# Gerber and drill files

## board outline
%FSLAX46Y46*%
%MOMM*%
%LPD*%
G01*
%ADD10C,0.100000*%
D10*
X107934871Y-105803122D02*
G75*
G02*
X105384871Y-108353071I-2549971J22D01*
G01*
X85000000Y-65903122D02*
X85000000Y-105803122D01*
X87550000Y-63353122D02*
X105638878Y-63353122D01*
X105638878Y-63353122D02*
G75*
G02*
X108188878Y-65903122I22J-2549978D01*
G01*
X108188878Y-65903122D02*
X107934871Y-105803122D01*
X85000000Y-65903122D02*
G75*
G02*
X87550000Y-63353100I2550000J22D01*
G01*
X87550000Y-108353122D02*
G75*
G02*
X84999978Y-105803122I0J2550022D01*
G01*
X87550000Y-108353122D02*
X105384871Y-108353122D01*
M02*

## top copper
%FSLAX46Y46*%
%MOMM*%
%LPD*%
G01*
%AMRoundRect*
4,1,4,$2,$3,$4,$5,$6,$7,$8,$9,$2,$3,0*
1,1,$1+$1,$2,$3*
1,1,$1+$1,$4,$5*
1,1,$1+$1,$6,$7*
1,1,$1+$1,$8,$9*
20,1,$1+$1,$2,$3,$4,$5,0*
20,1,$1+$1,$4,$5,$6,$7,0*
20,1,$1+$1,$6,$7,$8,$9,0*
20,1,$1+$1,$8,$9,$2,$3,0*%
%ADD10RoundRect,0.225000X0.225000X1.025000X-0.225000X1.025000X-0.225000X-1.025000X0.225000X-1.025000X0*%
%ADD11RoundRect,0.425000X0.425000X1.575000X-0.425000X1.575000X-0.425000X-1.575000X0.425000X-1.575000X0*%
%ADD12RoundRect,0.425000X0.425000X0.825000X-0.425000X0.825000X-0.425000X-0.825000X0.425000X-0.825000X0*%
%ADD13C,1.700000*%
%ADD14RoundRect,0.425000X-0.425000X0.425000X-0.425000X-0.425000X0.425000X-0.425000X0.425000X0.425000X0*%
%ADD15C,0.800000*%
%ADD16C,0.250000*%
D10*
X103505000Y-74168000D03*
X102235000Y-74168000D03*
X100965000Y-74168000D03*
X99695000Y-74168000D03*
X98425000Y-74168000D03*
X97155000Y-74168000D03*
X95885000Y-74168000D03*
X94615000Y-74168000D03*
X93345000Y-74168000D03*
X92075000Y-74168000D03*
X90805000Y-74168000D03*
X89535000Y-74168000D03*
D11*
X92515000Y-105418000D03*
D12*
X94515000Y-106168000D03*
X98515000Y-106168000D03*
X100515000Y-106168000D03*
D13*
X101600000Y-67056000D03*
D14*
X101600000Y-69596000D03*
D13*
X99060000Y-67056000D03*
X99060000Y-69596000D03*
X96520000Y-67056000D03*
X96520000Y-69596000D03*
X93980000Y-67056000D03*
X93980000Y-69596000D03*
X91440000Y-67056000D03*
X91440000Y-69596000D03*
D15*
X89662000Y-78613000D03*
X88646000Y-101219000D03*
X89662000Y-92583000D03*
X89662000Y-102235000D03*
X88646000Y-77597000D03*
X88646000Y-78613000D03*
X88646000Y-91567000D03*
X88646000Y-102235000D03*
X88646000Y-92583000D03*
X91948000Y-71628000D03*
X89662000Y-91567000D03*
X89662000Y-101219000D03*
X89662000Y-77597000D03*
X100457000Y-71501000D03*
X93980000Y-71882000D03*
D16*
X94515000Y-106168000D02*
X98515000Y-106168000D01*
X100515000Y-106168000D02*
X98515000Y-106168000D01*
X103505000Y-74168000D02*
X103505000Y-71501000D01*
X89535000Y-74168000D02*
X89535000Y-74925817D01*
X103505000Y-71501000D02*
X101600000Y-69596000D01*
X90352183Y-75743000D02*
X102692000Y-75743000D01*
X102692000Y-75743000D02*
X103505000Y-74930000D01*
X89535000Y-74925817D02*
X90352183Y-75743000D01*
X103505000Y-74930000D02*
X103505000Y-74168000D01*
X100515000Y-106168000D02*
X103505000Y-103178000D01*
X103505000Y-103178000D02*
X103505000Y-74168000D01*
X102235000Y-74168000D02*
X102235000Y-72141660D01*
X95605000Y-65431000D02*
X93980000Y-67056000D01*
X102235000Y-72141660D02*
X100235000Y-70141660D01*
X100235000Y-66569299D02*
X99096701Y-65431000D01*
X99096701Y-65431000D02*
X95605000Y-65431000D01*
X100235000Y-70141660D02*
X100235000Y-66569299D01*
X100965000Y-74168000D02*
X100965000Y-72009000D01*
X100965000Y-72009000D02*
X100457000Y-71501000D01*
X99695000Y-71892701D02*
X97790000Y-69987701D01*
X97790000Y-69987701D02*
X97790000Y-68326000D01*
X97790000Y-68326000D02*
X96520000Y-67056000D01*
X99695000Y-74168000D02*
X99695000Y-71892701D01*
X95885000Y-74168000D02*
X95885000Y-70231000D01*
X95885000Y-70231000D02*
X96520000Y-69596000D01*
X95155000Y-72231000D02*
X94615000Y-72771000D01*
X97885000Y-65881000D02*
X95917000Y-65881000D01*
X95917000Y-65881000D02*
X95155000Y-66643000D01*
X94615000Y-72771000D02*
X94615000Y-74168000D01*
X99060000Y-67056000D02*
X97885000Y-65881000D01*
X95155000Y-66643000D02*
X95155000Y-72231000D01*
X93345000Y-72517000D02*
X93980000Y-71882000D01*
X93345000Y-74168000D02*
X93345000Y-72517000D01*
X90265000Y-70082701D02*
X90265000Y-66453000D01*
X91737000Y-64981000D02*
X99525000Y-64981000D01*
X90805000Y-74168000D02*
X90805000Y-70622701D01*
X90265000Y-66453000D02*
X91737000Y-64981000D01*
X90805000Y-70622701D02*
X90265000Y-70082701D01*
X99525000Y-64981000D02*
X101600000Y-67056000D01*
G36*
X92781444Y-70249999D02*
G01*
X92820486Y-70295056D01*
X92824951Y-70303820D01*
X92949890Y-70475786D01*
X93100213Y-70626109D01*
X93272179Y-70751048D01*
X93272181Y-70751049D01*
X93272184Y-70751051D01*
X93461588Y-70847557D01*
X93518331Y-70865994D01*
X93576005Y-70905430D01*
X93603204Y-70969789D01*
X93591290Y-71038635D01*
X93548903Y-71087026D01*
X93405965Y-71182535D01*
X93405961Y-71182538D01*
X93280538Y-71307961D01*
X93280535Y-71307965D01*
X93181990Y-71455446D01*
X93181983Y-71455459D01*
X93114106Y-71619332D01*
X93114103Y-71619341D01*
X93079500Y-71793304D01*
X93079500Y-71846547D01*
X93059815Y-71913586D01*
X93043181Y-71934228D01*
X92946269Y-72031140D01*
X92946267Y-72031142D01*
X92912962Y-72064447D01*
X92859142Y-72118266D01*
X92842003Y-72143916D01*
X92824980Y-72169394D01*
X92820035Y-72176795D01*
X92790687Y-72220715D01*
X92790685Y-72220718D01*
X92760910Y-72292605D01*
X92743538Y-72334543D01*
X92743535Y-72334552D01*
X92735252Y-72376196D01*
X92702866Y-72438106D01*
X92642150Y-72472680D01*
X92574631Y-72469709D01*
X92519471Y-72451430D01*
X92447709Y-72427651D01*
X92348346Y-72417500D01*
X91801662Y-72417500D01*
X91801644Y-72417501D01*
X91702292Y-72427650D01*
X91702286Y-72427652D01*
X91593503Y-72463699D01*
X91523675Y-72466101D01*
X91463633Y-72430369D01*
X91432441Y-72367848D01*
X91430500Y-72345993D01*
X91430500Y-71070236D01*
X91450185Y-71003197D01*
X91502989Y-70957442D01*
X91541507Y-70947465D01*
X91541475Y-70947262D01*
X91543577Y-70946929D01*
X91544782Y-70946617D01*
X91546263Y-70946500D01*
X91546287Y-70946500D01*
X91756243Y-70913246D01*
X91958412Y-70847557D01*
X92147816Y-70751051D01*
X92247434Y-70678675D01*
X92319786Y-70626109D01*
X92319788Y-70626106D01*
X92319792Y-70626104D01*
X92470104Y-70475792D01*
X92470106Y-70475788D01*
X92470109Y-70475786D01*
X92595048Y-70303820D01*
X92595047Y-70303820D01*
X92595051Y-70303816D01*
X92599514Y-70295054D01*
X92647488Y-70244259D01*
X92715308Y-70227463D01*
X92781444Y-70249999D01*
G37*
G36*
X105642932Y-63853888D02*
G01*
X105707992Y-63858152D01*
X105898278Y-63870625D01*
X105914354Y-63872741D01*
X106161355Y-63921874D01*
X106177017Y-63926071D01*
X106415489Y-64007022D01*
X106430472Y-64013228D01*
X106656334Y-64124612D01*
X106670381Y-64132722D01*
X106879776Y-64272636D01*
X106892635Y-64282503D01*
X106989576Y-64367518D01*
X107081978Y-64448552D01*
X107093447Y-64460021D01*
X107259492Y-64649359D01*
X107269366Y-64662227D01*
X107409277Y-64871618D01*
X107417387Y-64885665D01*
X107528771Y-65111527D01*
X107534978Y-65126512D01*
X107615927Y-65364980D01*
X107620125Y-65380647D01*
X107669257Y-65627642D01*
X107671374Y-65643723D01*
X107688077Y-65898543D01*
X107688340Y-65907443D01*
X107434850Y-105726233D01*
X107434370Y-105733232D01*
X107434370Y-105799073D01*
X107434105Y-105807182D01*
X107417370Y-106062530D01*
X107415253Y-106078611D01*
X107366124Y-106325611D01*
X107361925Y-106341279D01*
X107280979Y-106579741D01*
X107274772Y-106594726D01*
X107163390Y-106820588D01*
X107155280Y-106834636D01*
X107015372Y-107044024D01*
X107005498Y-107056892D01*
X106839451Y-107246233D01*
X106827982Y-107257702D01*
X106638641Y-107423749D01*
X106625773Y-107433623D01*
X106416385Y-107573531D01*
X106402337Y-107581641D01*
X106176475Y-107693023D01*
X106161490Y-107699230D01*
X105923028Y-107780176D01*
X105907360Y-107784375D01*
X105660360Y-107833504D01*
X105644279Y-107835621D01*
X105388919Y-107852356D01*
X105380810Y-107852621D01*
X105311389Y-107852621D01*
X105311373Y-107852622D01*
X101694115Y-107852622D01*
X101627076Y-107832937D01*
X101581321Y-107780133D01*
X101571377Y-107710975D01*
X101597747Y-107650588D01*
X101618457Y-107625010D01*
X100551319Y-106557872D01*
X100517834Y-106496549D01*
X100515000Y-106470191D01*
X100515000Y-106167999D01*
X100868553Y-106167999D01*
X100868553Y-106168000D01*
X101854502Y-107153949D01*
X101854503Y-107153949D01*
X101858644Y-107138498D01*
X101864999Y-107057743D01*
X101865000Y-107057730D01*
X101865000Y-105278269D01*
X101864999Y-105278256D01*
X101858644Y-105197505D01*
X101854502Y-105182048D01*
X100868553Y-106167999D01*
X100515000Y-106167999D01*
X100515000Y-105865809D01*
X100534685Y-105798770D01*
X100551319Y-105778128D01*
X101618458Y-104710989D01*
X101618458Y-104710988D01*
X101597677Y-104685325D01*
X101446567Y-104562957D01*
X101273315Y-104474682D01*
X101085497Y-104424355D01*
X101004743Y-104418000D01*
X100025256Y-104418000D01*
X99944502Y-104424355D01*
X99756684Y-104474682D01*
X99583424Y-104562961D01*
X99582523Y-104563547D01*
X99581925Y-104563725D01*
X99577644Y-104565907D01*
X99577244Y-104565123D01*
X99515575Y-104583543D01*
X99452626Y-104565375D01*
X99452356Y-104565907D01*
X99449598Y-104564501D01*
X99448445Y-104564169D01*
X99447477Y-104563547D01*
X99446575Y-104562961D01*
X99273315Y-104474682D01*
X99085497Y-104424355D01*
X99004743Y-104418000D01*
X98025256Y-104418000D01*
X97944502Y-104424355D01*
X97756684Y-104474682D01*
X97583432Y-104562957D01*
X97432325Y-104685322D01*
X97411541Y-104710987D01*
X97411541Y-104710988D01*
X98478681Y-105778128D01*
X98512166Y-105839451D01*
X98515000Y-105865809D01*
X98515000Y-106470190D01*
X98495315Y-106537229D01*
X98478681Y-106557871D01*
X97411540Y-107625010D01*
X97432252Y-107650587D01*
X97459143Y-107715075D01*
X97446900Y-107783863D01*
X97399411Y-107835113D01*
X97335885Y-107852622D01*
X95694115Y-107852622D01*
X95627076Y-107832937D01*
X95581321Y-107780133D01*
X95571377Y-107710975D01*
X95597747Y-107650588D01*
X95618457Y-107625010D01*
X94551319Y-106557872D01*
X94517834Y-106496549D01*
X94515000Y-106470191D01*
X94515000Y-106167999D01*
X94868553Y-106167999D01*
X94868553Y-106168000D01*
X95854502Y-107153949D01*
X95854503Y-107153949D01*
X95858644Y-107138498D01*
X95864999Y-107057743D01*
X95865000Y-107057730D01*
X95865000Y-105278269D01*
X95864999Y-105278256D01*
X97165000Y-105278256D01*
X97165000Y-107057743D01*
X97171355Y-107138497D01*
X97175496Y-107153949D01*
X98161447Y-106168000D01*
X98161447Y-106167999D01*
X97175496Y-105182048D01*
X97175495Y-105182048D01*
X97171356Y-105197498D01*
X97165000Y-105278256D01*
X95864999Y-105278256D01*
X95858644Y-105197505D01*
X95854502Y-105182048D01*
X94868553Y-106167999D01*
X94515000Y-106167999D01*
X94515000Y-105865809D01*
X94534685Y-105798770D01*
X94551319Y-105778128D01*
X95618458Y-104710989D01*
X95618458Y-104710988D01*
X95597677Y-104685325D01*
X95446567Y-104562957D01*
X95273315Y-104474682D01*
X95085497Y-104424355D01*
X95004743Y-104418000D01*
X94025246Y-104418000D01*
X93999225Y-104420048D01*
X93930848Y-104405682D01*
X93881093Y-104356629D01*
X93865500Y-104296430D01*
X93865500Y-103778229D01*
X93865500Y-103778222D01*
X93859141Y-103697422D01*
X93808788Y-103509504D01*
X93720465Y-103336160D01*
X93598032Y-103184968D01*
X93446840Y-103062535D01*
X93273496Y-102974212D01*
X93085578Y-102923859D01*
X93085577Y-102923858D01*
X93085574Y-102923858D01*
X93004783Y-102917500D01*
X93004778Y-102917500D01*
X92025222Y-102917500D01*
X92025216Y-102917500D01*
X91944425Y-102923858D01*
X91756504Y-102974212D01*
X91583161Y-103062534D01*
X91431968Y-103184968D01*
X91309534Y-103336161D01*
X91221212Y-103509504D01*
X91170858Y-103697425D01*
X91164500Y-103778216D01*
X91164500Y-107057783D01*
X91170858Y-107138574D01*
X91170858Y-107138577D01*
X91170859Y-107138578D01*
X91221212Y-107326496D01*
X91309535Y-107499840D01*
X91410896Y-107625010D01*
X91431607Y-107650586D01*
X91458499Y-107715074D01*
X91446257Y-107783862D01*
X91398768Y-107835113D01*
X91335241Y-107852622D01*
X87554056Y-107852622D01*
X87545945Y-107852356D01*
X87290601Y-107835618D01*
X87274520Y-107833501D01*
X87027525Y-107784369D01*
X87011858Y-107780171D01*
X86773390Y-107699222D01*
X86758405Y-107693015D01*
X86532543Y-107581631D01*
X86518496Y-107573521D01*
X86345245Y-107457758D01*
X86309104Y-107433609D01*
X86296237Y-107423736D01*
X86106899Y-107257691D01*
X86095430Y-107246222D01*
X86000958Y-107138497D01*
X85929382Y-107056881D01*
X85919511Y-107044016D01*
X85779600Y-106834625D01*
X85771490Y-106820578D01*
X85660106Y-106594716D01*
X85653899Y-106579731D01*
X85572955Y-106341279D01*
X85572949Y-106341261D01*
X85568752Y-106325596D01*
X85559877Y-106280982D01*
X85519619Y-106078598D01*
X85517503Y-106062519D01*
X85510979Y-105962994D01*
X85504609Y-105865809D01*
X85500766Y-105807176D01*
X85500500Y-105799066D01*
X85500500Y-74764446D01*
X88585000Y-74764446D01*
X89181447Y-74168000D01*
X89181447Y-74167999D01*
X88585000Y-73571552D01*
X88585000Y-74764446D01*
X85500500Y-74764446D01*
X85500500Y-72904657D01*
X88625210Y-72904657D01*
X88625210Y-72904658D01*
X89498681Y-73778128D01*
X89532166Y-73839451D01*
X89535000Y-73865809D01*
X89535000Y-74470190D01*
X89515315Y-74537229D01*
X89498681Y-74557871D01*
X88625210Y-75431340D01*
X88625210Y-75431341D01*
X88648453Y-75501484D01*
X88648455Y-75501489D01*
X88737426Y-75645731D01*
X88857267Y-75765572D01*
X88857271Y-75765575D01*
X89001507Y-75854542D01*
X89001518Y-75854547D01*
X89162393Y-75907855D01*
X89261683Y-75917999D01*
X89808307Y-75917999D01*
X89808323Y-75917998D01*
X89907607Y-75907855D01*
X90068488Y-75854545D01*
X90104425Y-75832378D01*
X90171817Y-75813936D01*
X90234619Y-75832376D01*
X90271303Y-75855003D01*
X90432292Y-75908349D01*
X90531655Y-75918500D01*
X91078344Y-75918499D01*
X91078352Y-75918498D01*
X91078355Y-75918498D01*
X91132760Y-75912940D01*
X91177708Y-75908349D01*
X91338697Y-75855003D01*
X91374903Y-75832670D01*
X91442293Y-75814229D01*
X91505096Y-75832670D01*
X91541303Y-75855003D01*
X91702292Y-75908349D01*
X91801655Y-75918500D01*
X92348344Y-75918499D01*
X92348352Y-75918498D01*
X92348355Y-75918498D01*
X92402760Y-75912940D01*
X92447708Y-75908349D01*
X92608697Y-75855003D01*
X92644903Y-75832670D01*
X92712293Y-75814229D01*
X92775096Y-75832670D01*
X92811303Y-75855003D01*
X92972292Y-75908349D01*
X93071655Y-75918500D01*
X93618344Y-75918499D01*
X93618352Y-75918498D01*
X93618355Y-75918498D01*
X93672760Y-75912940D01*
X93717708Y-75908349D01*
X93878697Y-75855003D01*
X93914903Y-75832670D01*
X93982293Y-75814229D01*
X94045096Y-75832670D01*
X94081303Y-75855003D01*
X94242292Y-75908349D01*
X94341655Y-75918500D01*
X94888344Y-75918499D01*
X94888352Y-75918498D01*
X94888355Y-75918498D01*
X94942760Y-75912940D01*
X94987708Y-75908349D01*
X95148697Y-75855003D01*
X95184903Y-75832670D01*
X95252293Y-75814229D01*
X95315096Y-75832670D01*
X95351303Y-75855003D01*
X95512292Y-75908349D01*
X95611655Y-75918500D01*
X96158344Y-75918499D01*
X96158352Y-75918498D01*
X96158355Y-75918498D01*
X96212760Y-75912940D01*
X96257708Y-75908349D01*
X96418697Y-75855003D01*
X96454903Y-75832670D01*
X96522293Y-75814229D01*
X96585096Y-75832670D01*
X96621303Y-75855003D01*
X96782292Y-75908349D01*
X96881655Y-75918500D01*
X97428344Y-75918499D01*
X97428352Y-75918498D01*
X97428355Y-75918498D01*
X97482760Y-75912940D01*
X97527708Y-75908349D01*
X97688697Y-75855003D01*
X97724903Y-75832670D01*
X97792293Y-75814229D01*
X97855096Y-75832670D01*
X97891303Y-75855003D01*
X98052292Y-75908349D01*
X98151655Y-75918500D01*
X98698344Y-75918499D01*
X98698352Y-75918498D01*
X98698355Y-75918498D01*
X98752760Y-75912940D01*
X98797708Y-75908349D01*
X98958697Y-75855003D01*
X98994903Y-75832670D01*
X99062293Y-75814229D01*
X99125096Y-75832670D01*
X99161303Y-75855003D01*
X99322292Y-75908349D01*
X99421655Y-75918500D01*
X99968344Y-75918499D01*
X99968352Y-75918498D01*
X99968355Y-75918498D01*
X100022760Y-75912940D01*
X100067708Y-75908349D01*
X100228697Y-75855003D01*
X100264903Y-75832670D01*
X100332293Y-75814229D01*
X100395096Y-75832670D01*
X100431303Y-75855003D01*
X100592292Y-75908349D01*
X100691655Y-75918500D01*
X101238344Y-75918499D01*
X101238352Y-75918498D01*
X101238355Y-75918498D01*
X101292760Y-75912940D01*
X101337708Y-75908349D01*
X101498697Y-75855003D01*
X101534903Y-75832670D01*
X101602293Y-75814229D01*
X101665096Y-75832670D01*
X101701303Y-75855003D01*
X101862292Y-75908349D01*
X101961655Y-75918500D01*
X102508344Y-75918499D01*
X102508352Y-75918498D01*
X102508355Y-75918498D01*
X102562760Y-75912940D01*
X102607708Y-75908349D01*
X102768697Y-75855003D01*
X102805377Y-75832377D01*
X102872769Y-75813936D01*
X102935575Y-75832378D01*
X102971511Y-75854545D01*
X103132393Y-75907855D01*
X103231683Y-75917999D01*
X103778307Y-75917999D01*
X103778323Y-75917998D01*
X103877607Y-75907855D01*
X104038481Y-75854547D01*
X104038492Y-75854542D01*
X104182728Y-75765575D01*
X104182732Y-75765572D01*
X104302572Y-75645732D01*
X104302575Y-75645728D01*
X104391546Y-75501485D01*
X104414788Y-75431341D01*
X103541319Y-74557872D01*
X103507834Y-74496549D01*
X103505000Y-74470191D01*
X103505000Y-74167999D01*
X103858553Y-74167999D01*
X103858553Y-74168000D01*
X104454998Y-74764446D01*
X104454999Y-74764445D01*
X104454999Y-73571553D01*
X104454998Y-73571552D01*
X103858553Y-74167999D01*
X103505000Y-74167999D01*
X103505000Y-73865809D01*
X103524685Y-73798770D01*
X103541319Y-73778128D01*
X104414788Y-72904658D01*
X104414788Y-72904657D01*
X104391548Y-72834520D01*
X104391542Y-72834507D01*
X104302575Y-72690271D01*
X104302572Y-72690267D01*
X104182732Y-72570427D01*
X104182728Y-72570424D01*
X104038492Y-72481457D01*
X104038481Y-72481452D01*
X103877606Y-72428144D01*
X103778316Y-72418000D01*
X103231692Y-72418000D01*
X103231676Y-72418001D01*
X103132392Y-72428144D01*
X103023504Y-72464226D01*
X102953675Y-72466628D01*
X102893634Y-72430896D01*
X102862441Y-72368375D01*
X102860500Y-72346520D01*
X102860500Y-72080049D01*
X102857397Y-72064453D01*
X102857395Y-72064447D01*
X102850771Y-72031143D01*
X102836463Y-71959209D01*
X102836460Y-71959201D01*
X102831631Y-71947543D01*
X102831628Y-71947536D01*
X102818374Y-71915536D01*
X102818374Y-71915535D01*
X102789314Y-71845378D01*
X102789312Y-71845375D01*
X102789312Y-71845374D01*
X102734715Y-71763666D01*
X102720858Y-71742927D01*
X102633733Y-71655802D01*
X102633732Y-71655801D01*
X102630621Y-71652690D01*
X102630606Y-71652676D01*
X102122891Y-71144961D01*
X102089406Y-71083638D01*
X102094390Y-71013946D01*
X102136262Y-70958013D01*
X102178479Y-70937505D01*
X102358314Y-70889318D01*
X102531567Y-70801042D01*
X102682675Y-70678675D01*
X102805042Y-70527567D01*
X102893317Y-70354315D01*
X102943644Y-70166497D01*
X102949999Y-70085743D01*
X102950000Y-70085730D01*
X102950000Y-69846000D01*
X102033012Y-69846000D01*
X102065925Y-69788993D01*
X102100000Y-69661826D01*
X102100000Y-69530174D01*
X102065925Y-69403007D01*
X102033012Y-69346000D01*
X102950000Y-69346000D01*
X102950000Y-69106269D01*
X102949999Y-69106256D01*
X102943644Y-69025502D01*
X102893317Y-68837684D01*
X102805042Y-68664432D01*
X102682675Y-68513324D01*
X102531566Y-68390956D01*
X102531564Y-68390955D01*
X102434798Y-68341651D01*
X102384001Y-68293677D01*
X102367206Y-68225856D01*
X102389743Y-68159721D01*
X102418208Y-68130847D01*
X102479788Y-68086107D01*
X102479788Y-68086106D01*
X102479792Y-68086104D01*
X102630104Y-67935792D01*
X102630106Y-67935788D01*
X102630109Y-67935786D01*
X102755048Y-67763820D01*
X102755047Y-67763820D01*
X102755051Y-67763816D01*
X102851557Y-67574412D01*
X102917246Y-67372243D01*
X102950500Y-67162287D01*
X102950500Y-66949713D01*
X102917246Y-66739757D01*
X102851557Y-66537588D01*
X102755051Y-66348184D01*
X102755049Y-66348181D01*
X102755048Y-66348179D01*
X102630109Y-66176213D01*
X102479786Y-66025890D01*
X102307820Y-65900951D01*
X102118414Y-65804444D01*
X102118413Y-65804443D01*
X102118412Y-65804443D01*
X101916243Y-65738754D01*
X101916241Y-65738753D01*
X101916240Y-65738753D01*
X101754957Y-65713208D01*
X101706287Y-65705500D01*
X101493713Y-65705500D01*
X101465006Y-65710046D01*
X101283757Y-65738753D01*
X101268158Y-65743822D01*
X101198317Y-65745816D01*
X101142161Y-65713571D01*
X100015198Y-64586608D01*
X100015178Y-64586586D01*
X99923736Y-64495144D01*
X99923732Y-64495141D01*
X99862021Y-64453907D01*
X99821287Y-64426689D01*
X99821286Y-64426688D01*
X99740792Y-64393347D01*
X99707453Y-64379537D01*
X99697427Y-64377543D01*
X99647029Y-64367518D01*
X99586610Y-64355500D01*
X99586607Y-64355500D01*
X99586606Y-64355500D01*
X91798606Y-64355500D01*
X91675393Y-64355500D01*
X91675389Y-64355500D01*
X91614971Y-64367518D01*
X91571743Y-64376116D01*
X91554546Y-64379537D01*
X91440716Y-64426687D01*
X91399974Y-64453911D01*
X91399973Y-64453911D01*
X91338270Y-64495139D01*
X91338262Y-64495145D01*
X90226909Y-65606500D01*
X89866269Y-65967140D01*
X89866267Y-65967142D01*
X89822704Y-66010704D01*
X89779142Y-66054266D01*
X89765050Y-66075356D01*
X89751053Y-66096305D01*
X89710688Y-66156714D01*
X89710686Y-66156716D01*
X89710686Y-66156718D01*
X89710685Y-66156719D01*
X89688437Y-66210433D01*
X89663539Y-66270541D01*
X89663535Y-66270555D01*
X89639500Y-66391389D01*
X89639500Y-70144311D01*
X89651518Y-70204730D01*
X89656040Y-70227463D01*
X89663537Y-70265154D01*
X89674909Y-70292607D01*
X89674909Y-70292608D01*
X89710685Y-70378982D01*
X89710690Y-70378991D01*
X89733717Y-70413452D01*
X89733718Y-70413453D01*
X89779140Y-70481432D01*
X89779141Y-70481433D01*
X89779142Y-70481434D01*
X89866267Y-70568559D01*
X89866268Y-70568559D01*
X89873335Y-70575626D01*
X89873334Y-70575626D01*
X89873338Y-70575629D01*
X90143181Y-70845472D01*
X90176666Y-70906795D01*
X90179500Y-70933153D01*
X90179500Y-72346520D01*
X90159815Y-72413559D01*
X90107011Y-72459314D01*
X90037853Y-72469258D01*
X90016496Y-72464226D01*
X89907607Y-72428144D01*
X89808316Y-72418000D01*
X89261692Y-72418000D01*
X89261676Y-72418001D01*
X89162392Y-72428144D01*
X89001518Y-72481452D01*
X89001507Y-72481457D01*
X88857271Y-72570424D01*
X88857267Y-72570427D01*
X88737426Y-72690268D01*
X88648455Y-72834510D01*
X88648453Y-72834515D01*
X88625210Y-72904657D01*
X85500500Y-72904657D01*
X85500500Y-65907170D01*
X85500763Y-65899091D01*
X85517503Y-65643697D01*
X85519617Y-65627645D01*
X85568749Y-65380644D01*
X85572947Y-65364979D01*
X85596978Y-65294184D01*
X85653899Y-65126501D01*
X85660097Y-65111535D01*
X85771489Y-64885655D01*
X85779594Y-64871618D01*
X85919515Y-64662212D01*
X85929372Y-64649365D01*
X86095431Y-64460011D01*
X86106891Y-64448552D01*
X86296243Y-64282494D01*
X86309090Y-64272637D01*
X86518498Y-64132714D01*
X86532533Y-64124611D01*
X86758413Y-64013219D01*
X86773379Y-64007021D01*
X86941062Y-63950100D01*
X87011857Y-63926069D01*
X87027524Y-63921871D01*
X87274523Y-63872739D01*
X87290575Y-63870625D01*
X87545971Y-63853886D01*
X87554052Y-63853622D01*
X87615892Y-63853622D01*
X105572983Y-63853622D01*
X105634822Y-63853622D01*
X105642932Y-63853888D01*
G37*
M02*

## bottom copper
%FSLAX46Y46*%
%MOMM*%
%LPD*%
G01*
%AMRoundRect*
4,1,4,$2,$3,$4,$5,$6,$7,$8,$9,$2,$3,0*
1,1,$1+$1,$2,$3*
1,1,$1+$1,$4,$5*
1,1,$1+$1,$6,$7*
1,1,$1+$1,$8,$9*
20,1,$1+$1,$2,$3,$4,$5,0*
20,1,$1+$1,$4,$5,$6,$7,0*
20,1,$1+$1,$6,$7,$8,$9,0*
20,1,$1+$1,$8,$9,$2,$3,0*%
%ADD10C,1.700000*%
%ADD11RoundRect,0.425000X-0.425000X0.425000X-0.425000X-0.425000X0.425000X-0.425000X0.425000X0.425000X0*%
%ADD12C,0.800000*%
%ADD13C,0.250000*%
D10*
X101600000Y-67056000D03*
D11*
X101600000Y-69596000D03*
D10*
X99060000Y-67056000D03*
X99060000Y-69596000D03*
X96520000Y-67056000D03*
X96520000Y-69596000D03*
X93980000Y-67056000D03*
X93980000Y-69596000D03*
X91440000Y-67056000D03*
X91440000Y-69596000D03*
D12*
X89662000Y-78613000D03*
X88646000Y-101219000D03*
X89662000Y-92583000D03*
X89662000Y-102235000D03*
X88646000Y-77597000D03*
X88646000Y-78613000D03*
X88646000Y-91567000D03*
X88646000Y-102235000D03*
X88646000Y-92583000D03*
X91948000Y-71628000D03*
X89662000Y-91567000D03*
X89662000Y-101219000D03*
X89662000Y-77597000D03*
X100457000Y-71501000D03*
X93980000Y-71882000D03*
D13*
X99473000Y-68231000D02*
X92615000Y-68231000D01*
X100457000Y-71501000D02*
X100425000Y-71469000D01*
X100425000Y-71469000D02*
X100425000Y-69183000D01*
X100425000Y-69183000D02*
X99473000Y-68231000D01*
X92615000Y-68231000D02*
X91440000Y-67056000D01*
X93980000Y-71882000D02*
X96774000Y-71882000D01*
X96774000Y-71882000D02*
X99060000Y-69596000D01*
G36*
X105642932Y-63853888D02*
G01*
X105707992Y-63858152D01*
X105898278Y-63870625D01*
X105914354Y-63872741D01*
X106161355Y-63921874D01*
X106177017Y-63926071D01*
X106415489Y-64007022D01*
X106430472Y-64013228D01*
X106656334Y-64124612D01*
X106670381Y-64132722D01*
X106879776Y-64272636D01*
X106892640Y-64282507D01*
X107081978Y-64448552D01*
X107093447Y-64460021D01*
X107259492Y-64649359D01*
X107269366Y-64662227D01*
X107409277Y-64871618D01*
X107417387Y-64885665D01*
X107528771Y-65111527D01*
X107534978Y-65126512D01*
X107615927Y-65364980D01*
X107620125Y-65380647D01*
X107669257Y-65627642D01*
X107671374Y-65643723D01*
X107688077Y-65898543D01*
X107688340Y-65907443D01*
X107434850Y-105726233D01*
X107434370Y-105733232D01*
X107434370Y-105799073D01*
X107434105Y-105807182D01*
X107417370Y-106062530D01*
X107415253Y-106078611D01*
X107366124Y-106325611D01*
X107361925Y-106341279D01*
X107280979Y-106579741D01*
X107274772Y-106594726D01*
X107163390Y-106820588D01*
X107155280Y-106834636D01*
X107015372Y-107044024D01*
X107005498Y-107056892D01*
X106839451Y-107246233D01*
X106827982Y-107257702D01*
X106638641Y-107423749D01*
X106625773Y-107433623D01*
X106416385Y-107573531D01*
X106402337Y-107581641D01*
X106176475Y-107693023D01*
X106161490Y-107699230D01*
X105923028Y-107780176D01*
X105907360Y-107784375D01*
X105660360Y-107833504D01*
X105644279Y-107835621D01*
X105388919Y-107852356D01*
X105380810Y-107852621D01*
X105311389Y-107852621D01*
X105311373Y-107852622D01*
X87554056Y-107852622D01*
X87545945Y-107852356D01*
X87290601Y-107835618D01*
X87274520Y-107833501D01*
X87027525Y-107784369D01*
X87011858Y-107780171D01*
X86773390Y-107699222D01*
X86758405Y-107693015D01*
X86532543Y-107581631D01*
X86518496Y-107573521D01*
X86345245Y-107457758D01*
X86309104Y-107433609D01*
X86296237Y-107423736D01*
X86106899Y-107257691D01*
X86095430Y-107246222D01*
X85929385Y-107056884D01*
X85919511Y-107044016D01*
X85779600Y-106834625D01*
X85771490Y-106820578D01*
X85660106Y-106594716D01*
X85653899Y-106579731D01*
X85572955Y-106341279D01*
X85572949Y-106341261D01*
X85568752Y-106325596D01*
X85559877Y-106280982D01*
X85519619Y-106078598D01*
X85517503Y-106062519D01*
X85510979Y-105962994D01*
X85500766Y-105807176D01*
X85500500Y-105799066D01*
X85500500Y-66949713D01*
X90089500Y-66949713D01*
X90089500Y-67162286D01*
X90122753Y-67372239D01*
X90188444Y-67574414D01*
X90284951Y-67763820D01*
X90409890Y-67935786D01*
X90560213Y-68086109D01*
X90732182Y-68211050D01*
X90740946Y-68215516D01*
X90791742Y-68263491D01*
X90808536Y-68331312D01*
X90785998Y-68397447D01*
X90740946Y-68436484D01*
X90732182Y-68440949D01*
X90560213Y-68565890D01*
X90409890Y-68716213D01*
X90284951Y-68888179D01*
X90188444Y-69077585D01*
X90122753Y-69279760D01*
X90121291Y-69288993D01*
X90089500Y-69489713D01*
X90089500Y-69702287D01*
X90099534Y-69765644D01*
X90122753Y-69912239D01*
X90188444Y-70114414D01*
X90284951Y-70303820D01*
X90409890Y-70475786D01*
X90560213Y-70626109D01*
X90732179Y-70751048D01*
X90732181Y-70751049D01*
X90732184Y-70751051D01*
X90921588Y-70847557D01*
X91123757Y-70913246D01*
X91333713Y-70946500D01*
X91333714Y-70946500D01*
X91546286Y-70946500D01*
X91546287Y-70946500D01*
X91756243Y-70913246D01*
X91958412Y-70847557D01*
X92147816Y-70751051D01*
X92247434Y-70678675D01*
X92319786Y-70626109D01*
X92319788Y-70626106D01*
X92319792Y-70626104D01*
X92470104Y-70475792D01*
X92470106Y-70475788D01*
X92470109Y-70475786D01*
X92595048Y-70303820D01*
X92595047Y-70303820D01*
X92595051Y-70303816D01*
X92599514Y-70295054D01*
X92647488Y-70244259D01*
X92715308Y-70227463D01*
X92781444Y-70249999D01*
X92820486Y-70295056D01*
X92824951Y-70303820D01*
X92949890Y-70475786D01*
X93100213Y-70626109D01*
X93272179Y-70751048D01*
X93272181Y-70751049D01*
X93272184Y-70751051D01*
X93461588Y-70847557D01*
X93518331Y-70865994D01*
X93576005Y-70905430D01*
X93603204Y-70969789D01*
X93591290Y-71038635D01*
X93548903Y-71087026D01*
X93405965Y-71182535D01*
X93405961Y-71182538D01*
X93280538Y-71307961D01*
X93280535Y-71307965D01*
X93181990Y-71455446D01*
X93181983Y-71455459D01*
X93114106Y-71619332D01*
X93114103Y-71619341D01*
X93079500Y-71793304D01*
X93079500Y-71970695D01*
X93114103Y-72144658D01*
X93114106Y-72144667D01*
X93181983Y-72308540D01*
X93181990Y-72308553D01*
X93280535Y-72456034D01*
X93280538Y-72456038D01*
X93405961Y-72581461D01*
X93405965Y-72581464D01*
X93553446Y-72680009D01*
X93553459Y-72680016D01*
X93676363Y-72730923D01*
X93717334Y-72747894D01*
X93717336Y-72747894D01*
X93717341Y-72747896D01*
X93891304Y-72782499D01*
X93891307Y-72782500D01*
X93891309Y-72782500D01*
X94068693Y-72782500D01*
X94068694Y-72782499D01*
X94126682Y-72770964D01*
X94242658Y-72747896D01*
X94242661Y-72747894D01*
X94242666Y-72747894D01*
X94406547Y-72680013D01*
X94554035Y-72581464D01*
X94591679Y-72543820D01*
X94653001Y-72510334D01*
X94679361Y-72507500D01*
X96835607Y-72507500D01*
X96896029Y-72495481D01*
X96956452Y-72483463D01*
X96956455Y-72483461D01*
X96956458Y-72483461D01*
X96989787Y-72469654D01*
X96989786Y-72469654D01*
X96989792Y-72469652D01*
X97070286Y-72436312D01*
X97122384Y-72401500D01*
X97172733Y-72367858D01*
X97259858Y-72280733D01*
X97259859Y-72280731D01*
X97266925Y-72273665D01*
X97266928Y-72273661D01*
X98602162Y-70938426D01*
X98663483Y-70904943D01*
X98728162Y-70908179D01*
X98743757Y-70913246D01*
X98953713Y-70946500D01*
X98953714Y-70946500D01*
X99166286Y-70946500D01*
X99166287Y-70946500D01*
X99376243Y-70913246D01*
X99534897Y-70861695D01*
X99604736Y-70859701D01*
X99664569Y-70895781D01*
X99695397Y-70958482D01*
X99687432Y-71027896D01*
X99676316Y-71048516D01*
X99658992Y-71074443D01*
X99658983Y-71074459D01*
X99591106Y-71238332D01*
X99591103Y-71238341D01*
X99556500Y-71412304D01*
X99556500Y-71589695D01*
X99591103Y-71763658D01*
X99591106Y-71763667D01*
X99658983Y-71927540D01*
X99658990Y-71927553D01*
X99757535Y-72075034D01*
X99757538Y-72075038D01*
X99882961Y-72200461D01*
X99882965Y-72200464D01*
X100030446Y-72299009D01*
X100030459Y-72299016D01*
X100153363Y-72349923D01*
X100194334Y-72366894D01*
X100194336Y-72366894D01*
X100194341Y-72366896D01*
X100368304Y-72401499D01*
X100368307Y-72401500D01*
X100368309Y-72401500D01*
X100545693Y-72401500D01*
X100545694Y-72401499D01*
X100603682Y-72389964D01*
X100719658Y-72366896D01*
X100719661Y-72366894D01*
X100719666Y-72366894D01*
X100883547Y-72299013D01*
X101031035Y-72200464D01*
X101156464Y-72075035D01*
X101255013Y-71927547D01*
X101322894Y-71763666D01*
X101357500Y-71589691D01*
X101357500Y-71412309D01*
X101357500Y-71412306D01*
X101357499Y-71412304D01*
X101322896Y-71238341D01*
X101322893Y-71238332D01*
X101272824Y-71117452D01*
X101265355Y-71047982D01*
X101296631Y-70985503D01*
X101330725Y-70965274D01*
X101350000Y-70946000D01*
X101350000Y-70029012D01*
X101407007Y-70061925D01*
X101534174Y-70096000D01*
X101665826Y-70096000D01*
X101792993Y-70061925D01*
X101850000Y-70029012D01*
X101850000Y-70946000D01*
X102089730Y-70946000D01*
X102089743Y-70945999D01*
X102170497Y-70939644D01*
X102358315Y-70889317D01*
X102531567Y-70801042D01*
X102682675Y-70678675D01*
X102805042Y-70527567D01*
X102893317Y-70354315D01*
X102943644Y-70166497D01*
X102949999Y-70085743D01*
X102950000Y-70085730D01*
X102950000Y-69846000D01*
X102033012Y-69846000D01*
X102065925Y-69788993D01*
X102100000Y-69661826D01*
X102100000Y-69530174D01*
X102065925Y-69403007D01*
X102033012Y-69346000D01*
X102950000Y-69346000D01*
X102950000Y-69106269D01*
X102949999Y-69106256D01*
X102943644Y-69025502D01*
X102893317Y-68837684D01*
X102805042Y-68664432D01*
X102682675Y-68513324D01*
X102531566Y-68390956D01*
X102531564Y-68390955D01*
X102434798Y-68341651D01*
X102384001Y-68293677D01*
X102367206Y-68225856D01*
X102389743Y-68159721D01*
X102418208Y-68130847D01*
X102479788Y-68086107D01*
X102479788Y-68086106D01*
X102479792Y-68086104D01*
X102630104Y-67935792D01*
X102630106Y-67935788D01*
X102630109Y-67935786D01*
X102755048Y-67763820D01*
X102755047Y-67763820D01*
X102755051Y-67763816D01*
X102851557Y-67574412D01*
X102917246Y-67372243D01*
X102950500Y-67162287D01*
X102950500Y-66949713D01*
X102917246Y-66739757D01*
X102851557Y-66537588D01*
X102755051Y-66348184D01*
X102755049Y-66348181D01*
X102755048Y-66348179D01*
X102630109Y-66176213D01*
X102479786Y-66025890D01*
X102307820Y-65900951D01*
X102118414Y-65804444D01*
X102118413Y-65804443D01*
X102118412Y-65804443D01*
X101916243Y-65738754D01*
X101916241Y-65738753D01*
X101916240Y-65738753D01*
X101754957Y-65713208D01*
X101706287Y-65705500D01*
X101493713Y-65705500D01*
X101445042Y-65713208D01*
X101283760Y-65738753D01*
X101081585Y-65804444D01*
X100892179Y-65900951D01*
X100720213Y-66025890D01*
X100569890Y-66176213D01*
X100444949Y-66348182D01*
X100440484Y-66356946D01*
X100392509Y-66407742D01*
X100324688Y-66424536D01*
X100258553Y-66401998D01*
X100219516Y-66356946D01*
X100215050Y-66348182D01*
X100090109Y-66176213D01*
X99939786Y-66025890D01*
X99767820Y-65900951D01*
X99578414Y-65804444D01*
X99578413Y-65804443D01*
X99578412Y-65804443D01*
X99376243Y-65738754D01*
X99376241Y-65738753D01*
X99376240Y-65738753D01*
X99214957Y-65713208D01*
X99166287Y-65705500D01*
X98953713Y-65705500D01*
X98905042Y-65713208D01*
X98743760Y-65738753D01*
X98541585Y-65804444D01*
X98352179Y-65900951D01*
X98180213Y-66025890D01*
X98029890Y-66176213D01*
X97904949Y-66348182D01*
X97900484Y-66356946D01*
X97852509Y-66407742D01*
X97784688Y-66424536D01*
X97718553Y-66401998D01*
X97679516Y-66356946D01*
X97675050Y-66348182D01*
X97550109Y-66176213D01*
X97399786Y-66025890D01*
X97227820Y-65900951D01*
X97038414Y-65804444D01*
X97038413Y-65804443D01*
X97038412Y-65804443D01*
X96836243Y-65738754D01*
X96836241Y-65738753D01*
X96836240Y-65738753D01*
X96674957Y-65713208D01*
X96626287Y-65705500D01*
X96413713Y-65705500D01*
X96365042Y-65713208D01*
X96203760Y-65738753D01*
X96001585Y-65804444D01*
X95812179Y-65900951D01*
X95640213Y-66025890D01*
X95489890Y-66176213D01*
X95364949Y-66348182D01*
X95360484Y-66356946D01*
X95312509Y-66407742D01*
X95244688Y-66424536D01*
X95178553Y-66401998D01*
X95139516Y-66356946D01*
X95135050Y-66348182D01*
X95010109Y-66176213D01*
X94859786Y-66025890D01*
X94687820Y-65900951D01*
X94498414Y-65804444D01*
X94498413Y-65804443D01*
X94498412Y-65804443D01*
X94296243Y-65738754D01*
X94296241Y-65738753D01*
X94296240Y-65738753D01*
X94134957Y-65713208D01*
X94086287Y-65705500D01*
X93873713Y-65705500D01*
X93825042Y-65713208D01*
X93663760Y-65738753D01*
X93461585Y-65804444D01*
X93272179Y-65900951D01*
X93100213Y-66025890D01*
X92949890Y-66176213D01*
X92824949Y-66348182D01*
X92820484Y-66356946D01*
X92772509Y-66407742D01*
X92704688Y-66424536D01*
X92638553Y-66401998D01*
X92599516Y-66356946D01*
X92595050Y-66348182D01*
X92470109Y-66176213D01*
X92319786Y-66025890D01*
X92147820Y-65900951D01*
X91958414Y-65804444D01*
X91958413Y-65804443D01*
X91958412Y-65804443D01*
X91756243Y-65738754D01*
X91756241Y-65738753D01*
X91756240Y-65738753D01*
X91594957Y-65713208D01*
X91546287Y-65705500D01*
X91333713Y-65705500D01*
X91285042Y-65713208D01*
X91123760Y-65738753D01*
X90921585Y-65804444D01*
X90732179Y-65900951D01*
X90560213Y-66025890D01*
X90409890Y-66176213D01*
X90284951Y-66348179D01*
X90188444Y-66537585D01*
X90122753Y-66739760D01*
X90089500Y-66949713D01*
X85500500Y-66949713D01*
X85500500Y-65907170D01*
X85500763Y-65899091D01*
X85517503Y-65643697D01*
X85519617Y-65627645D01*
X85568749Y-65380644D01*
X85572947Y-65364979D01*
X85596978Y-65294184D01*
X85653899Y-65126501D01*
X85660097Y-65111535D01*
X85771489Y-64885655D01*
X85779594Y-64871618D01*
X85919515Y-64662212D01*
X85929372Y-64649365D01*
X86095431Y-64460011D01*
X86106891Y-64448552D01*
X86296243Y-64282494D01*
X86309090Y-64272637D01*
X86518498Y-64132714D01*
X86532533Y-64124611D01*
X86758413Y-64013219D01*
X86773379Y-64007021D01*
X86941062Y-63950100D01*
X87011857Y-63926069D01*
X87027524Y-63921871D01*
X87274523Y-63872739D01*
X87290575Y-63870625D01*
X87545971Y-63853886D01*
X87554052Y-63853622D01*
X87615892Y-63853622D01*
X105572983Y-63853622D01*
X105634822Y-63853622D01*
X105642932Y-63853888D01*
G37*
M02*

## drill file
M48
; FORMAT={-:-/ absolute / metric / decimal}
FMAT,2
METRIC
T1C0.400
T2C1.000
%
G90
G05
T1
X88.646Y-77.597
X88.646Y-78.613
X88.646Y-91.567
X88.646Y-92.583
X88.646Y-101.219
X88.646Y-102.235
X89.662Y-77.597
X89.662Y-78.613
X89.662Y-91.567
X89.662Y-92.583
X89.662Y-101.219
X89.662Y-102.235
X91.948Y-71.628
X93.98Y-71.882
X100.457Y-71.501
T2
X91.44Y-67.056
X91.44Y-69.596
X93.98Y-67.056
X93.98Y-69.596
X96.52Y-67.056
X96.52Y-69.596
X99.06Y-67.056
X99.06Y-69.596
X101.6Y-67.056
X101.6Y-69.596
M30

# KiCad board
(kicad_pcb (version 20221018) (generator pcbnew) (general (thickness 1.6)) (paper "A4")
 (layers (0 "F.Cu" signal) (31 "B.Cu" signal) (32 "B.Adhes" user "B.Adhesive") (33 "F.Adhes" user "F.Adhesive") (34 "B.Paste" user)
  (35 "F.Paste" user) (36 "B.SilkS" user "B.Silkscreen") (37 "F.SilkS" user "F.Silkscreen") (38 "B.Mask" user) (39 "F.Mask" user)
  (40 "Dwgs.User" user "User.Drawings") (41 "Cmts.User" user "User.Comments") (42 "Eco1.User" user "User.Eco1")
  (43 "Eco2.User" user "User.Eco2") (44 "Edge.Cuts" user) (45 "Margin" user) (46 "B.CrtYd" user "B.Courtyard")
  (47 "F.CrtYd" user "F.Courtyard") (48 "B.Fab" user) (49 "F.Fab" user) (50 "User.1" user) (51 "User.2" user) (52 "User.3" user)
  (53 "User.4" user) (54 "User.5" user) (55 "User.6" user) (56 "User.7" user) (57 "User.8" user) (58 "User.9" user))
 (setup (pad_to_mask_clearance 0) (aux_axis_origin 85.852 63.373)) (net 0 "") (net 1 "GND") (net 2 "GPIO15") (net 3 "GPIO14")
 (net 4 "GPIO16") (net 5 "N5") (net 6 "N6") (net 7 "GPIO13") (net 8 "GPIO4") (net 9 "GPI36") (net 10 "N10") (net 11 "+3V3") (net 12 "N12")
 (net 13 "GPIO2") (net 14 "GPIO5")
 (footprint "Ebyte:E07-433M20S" (layer "F.Cu") (at 87.515 106.168)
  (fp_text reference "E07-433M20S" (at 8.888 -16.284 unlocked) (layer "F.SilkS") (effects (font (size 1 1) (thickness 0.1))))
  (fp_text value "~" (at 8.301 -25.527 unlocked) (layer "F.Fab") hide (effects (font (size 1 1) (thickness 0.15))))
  (pad "1" smd roundrect (at 15.99 -32 180) (size 0.9 2.5) (layers "F.Cu" "F.Paste" "F.Mask") (roundrect_rratio 0.25) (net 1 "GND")
   (thermal_bridge_angle 45))
  (pad "2" smd roundrect (at 14.72 -32 180) (size 0.9 2.5) (layers "F.Cu" "F.Paste" "F.Mask") (roundrect_rratio 0.25) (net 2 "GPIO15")
   (thermal_bridge_angle 45))
  (pad "3" smd roundrect (at 13.45 -32 180) (size 0.9 2.5) (layers "F.Cu" "F.Paste" "F.Mask") (roundrect_rratio 0.25) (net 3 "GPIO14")
   (thermal_bridge_angle 45))
  (pad "4" smd roundrect (at 12.18 -32 180) (size 0.9 2.5) (layers "F.Cu" "F.Paste" "F.Mask") (roundrect_rratio 0.25) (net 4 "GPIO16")
   (thermal_bridge_angle 45))
  (pad "5" smd roundrect (at 10.91 -32 180) (size 0.9 2.5) (layers "F.Cu" "F.Paste" "F.Mask") (roundrect_rratio 0.25) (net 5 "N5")
   (thermal_bridge_angle 45))
  (pad "6" smd roundrect (at 9.64 -32 180) (size 0.9 2.5) (layers "F.Cu" "F.Paste" "F.Mask") (roundrect_rratio 0.25) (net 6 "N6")
   (thermal_bridge_angle 45))
  (pad "7" smd roundrect (at 8.37 -32 180) (size 0.9 2.5) (layers "F.Cu" "F.Paste" "F.Mask") (roundrect_rratio 0.25) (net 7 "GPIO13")
   (thermal_bridge_angle 45))
  (pad "8" smd roundrect (at 7.1 -32 180) (size 0.9 2.5) (layers "F.Cu" "F.Paste" "F.Mask") (roundrect_rratio 0.25) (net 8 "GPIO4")
   (thermal_bridge_angle 45))
  (pad "9" smd roundrect (at 5.83 -32 180) (size 0.9 2.5) (layers "F.Cu" "F.Paste" "F.Mask") (roundrect_rratio 0.25) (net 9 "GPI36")
   (thermal_bridge_angle 45))
  (pad "10" smd roundrect (at 4.56 -32 180) (size 0.9 2.5) (layers "F.Cu" "F.Paste" "F.Mask") (roundrect_rratio 0.25) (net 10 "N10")
   (thermal_bridge_angle 45))
  (pad "11" smd roundrect (at 3.29 -32 180) (size 0.9 2.5) (layers "F.Cu" "F.Paste" "F.Mask") (roundrect_rratio 0.25) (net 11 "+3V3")
   (thermal_bridge_angle 45))
  (pad "12" smd roundrect (at 2.02 -32 180) (size 0.9 2.5) (layers "F.Cu" "F.Paste" "F.Mask") (roundrect_rratio 0.25) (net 1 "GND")
   (thermal_bridge_angle 45))
  (pad "13" smd roundrect (at 5 -0.75 180) (size 1.7 4) (layers "F.Cu" "F.Paste" "F.Mask") (roundrect_rratio 0.25) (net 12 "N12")
   (thermal_bridge_angle 45))
  (pad "14" smd roundrect (at 7 0 180) (size 1.7 2.5) (layers "F.Cu" "F.Paste" "F.Mask") (roundrect_rratio 0.25) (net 1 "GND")
   (thermal_bridge_angle 45))
  (pad "15" smd roundrect (at 11 0 180) (size 1.7 2.5) (layers "F.Cu" "F.Paste" "F.Mask") (roundrect_rratio 0.25) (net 1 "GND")
   (thermal_bridge_angle 45))
  (pad "16" smd roundrect (at 13 0 180) (size 1.7 2.5) (layers "F.Cu" "F.Paste" "F.Mask") (roundrect_rratio 0.25) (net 1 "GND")
   (thermal_bridge_angle 45)))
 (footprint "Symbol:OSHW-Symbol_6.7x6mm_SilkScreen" (layer "F.Cu") (at 96.393 83.693)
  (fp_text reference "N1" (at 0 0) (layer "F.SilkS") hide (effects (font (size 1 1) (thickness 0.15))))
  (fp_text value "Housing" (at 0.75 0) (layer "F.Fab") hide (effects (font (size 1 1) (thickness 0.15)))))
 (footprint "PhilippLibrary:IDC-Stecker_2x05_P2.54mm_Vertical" (layer "B.Cu") (at 91.44 67.056 -90)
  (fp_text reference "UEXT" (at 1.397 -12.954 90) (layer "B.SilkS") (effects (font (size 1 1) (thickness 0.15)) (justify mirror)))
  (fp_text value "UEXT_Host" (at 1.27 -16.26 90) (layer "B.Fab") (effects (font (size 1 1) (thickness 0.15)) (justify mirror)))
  (pad "1" thru_hole circle (at 0 -10.16 270) (size 1.7 1.7) (drill 1) (layers "*.Cu" "*.Mask") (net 11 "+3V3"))
  (pad "2" thru_hole roundrect (at 2.54 -10.16 270) (size 1.7 1.7) (drill 1) (layers "*.Cu" "*.Mask") (roundrect_rratio 0.25) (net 1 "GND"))
  (pad "3" thru_hole circle (at 0 -7.62 270) (size 1.7 1.7) (drill 1) (layers "*.Cu" "*.Mask") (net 8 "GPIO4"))
  (pad "4" thru_hole circle (at 2.54 -7.62 270) (size 1.7 1.7) (drill 1) (layers "*.Cu" "*.Mask") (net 9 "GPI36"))
  (pad "5" thru_hole circle (at 0 -5.08 270) (size 1.7 1.7) (drill 1) (layers "*.Cu" "*.Mask") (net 4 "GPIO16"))
  (pad "6" thru_hole circle (at 2.54 -5.08 270) (size 1.7 1.7) (drill 1) (layers "*.Cu" "*.Mask") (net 7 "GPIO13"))
  (pad "7" thru_hole circle (at 0 -2.54 270) (size 1.7 1.7) (drill 1) (layers "*.Cu" "*.Mask") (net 2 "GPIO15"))
  (pad "8" thru_hole circle (at 2.54 -2.54 270) (size 1.7 1.7) (drill 1) (layers "*.Cu" "*.Mask") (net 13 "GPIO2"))
  (pad "9" thru_hole circle (at 0 0 270) (size 1.7 1.7) (drill 1) (layers "*.Cu" "*.Mask") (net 3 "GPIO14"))
  (pad "10" thru_hole circle (at 2.54 0 270) (size 1.7 1.7) (drill 1) (layers "*.Cu" "*.Mask") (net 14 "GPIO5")))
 (gr_arc (start 107.934871 105.803122) (mid 107.188 107.606251) (end 105.384871 108.353122) (stroke (width 0.1) (type default))
  (layer "Edge.Cuts"))
 (gr_line (start 85 65.903122) (end 85 105.803122) (stroke (width 0.1) (type default)) (layer "Edge.Cuts"))
 (gr_line (start 87.55 63.353122) (end 105.638878 63.353122) (stroke (width 0.1) (type default)) (layer "Edge.Cuts"))
 (gr_arc (start 105.638878 63.353122) (mid 107.441993 64.100001) (end 108.188878 65.903122) (stroke (width 0.1) (type default))
  (layer "Edge.Cuts"))
 (gr_line (start 108.188878 65.903122) (end 107.934871 105.803122) (stroke (width 0.1) (type default)) (layer "Edge.Cuts"))
 (gr_arc (start 85 65.903122) (mid 85.746878 64.1) (end 87.55 63.353122) (stroke (width 0.1) (type default)) (layer "Edge.Cuts"))
 (gr_arc (start 87.55 108.353122) (mid 85.746885 107.606243) (end 85 105.803122) (stroke (width 0.1) (type default)) (layer "Edge.Cuts"))
 (gr_line (start 87.55 108.353122) (end 105.384871 108.353122) (stroke (width 0.1) (type default)) (layer "Edge.Cuts"))
 (segment (start 94.515 106.168) (end 98.515 106.168) (width 0.25) (layer "F.Cu") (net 1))
 (segment (start 100.515 106.168) (end 98.515 106.168) (width 0.25) (layer "F.Cu") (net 1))
 (segment (start 103.505 74.168) (end 103.505 71.501) (width 0.25) (layer "F.Cu") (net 1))
 (segment (start 89.535 74.168) (end 89.535 74.925817) (width 0.25) (layer "F.Cu") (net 1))
 (segment (start 103.505 71.501) (end 101.6 69.596) (width 0.25) (layer "F.Cu") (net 1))
 (segment (start 90.352183 75.743) (end 102.692 75.743) (width 0.25) (layer "F.Cu") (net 1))
 (segment (start 102.692 75.743) (end 103.505 74.93) (width 0.25) (layer "F.Cu") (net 1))
 (segment (start 89.535 74.925817) (end 90.352183 75.743) (width 0.25) (layer "F.Cu") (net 1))
 (segment (start 103.505 74.93) (end 103.505 74.168) (width 0.25) (layer "F.Cu") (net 1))
 (segment (start 100.515 106.168) (end 103.505 103.178) (width 0.25) (layer "F.Cu") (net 1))
 (segment (start 103.505 103.178) (end 103.505 74.168) (width 0.25) (layer "F.Cu") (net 1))
 (via (at 89.662 78.613) (size 0.8) (drill 0.4) (layers "F.Cu" "B.Cu") (free) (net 1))
 (via (at 88.646 101.219) (size 0.8) (drill 0.4) (layers "F.Cu" "B.Cu") (free) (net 1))
 (via (at 89.662 92.583) (size 0.8) (drill 0.4) (layers "F.Cu" "B.Cu") (free) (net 1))
 (via (at 89.662 102.235) (size 0.8) (drill 0.4) (layers "F.Cu" "B.Cu") (free) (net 1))
 (via (at 88.646 77.597) (size 0.8) (drill 0.4) (layers "F.Cu" "B.Cu") (free) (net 1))
 (via (at 88.646 78.613) (size 0.8) (drill 0.4) (layers "F.Cu" "B.Cu") (free) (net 1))
 (via (at 88.646 91.567) (size 0.8) (drill 0.4) (layers "F.Cu" "B.Cu") (free) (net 1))
 (via (at 88.646 102.235) (size 0.8) (drill 0.4) (layers "F.Cu" "B.Cu") (free) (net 1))
 (via (at 88.646 92.583) (size 0.8) (drill 0.4) (layers "F.Cu" "B.Cu") (free) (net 1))
 (via (at 91.948 71.628) (size 0.8) (drill 0.4) (layers "F.Cu" "B.Cu") (free) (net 1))
 (via (at 89.662 91.567) (size 0.8) (drill 0.4) (layers "F.Cu" "B.Cu") (free) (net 1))
 (via (at 89.662 101.219) (size 0.8) (drill 0.4) (layers "F.Cu" "B.Cu") (free) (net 1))
 (via (at 89.662 77.597) (size 0.8) (drill 0.4) (layers "F.Cu" "B.Cu") (free) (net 1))
 (segment (start 102.235 74.168) (end 102.235 72.14166) (width 0.25) (layer "F.Cu") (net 2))
 (segment (start 95.605 65.431) (end 93.98 67.056) (width 0.25) (layer "F.Cu") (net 2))
 (segment (start 102.235 72.14166) (end 100.235 70.14166) (width 0.25) (layer "F.Cu") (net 2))
 (segment (start 100.235 66.569299) (end 99.096701 65.431) (width 0.25) (layer "F.Cu") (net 2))
 (segment (start 99.096701 65.431) (end 95.605 65.431) (width 0.25) (layer "F.Cu") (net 2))
 (segment (start 100.235 70.14166) (end 100.235 66.569299) (width 0.25) (layer "F.Cu") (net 2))
 (segment (start 100.965 74.168) (end 100.965 72.009) (width 0.25) (layer "F.Cu") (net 3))
 (segment (start 100.965 72.009) (end 100.457 71.501) (width 0.25) (layer "F.Cu") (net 3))
 (via (at 100.457 71.501) (size 0.8) (drill 0.4) (layers "F.Cu" "B.Cu") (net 3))
 (segment (start 99.473 68.231) (end 92.615 68.231) (width 0.25) (layer "B.Cu") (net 3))
 (segment (start 100.457 71.501) (end 100.425 71.469) (width 0.25) (layer "B.Cu") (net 3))
 (segment (start 100.425 71.469) (end 100.425 69.183) (width 0.25) (layer "B.Cu") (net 3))
 (segment (start 100.425 69.183) (end 99.473 68.231) (width 0.25) (layer "B.Cu") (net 3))
 (segment (start 92.615 68.231) (end 91.44 67.056) (width 0.25) (layer "B.Cu") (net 3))
 (segment (start 99.695 71.892701) (end 97.79 69.987701) (width 0.25) (layer "F.Cu") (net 4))
 (segment (start 97.79 69.987701) (end 97.79 68.326) (width 0.25) (layer "F.Cu") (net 4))
 (segment (start 97.79 68.326) (end 96.52 67.056) (width 0.25) (layer "F.Cu") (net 4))
 (segment (start 99.695 74.168) (end 99.695 71.892701) (width 0.25) (layer "F.Cu") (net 4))
 (segment (start 95.885 74.168) (end 95.885 70.231) (width 0.25) (layer "F.Cu") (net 7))
 (segment (start 95.885 70.231) (end 96.52 69.596) (width 0.25) (layer "F.Cu") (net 7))
 (segment (start 95.155 72.231) (end 94.615 72.771) (width 0.25) (layer "F.Cu") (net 8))
 (segment (start 97.885 65.881) (end 95.917 65.881) (width 0.25) (layer "F.Cu") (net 8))
 (segment (start 95.917 65.881) (end 95.155 66.643) (width 0.25) (layer "F.Cu") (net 8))
 (segment (start 94.615 72.771) (end 94.615 74.168) (width 0.25) (layer "F.Cu") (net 8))
 (segment (start 99.06 67.056) (end 97.885 65.881) (width 0.25) (layer "F.Cu") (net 8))
 (segment (start 95.155 66.643) (end 95.155 72.231) (width 0.25) (layer "F.Cu") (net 8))
 (segment (start 93.345 72.517) (end 93.98 71.882) (width 0.25) (layer "F.Cu") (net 9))
 (segment (start 93.345 74.168) (end 93.345 72.517) (width 0.25) (layer "F.Cu") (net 9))
 (via (at 93.98 71.882) (size 0.8) (drill 0.4) (layers "F.Cu" "B.Cu") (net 9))
 (segment (start 93.98 71.882) (end 96.774 71.882) (width 0.25) (layer "B.Cu") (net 9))
 (segment (start 96.774 71.882) (end 99.06 69.596) (width 0.25) (layer "B.Cu") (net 9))
 (segment (start 90.265 70.082701) (end 90.265 66.453) (width 0.25) (layer "F.Cu") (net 11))
 (segment (start 91.737 64.981) (end 99.525 64.981) (width 0.25) (layer "F.Cu") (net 11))
 (segment (start 90.805 74.168) (end 90.805 70.622701) (width 0.25) (layer "F.Cu") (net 11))
 (segment (start 90.265 66.453) (end 91.737 64.981) (width 0.25) (layer "F.Cu") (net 11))
 (segment (start 90.805 70.622701) (end 90.265 70.082701) (width 0.25) (layer "F.Cu") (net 11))
 (segment (start 99.525 64.981) (end 101.6 67.056) (width 0.25) (layer "F.Cu") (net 11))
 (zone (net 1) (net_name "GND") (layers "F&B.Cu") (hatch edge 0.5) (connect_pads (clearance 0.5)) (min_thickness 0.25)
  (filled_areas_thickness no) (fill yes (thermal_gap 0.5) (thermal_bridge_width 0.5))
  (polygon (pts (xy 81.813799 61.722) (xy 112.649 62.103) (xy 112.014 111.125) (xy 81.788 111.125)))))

